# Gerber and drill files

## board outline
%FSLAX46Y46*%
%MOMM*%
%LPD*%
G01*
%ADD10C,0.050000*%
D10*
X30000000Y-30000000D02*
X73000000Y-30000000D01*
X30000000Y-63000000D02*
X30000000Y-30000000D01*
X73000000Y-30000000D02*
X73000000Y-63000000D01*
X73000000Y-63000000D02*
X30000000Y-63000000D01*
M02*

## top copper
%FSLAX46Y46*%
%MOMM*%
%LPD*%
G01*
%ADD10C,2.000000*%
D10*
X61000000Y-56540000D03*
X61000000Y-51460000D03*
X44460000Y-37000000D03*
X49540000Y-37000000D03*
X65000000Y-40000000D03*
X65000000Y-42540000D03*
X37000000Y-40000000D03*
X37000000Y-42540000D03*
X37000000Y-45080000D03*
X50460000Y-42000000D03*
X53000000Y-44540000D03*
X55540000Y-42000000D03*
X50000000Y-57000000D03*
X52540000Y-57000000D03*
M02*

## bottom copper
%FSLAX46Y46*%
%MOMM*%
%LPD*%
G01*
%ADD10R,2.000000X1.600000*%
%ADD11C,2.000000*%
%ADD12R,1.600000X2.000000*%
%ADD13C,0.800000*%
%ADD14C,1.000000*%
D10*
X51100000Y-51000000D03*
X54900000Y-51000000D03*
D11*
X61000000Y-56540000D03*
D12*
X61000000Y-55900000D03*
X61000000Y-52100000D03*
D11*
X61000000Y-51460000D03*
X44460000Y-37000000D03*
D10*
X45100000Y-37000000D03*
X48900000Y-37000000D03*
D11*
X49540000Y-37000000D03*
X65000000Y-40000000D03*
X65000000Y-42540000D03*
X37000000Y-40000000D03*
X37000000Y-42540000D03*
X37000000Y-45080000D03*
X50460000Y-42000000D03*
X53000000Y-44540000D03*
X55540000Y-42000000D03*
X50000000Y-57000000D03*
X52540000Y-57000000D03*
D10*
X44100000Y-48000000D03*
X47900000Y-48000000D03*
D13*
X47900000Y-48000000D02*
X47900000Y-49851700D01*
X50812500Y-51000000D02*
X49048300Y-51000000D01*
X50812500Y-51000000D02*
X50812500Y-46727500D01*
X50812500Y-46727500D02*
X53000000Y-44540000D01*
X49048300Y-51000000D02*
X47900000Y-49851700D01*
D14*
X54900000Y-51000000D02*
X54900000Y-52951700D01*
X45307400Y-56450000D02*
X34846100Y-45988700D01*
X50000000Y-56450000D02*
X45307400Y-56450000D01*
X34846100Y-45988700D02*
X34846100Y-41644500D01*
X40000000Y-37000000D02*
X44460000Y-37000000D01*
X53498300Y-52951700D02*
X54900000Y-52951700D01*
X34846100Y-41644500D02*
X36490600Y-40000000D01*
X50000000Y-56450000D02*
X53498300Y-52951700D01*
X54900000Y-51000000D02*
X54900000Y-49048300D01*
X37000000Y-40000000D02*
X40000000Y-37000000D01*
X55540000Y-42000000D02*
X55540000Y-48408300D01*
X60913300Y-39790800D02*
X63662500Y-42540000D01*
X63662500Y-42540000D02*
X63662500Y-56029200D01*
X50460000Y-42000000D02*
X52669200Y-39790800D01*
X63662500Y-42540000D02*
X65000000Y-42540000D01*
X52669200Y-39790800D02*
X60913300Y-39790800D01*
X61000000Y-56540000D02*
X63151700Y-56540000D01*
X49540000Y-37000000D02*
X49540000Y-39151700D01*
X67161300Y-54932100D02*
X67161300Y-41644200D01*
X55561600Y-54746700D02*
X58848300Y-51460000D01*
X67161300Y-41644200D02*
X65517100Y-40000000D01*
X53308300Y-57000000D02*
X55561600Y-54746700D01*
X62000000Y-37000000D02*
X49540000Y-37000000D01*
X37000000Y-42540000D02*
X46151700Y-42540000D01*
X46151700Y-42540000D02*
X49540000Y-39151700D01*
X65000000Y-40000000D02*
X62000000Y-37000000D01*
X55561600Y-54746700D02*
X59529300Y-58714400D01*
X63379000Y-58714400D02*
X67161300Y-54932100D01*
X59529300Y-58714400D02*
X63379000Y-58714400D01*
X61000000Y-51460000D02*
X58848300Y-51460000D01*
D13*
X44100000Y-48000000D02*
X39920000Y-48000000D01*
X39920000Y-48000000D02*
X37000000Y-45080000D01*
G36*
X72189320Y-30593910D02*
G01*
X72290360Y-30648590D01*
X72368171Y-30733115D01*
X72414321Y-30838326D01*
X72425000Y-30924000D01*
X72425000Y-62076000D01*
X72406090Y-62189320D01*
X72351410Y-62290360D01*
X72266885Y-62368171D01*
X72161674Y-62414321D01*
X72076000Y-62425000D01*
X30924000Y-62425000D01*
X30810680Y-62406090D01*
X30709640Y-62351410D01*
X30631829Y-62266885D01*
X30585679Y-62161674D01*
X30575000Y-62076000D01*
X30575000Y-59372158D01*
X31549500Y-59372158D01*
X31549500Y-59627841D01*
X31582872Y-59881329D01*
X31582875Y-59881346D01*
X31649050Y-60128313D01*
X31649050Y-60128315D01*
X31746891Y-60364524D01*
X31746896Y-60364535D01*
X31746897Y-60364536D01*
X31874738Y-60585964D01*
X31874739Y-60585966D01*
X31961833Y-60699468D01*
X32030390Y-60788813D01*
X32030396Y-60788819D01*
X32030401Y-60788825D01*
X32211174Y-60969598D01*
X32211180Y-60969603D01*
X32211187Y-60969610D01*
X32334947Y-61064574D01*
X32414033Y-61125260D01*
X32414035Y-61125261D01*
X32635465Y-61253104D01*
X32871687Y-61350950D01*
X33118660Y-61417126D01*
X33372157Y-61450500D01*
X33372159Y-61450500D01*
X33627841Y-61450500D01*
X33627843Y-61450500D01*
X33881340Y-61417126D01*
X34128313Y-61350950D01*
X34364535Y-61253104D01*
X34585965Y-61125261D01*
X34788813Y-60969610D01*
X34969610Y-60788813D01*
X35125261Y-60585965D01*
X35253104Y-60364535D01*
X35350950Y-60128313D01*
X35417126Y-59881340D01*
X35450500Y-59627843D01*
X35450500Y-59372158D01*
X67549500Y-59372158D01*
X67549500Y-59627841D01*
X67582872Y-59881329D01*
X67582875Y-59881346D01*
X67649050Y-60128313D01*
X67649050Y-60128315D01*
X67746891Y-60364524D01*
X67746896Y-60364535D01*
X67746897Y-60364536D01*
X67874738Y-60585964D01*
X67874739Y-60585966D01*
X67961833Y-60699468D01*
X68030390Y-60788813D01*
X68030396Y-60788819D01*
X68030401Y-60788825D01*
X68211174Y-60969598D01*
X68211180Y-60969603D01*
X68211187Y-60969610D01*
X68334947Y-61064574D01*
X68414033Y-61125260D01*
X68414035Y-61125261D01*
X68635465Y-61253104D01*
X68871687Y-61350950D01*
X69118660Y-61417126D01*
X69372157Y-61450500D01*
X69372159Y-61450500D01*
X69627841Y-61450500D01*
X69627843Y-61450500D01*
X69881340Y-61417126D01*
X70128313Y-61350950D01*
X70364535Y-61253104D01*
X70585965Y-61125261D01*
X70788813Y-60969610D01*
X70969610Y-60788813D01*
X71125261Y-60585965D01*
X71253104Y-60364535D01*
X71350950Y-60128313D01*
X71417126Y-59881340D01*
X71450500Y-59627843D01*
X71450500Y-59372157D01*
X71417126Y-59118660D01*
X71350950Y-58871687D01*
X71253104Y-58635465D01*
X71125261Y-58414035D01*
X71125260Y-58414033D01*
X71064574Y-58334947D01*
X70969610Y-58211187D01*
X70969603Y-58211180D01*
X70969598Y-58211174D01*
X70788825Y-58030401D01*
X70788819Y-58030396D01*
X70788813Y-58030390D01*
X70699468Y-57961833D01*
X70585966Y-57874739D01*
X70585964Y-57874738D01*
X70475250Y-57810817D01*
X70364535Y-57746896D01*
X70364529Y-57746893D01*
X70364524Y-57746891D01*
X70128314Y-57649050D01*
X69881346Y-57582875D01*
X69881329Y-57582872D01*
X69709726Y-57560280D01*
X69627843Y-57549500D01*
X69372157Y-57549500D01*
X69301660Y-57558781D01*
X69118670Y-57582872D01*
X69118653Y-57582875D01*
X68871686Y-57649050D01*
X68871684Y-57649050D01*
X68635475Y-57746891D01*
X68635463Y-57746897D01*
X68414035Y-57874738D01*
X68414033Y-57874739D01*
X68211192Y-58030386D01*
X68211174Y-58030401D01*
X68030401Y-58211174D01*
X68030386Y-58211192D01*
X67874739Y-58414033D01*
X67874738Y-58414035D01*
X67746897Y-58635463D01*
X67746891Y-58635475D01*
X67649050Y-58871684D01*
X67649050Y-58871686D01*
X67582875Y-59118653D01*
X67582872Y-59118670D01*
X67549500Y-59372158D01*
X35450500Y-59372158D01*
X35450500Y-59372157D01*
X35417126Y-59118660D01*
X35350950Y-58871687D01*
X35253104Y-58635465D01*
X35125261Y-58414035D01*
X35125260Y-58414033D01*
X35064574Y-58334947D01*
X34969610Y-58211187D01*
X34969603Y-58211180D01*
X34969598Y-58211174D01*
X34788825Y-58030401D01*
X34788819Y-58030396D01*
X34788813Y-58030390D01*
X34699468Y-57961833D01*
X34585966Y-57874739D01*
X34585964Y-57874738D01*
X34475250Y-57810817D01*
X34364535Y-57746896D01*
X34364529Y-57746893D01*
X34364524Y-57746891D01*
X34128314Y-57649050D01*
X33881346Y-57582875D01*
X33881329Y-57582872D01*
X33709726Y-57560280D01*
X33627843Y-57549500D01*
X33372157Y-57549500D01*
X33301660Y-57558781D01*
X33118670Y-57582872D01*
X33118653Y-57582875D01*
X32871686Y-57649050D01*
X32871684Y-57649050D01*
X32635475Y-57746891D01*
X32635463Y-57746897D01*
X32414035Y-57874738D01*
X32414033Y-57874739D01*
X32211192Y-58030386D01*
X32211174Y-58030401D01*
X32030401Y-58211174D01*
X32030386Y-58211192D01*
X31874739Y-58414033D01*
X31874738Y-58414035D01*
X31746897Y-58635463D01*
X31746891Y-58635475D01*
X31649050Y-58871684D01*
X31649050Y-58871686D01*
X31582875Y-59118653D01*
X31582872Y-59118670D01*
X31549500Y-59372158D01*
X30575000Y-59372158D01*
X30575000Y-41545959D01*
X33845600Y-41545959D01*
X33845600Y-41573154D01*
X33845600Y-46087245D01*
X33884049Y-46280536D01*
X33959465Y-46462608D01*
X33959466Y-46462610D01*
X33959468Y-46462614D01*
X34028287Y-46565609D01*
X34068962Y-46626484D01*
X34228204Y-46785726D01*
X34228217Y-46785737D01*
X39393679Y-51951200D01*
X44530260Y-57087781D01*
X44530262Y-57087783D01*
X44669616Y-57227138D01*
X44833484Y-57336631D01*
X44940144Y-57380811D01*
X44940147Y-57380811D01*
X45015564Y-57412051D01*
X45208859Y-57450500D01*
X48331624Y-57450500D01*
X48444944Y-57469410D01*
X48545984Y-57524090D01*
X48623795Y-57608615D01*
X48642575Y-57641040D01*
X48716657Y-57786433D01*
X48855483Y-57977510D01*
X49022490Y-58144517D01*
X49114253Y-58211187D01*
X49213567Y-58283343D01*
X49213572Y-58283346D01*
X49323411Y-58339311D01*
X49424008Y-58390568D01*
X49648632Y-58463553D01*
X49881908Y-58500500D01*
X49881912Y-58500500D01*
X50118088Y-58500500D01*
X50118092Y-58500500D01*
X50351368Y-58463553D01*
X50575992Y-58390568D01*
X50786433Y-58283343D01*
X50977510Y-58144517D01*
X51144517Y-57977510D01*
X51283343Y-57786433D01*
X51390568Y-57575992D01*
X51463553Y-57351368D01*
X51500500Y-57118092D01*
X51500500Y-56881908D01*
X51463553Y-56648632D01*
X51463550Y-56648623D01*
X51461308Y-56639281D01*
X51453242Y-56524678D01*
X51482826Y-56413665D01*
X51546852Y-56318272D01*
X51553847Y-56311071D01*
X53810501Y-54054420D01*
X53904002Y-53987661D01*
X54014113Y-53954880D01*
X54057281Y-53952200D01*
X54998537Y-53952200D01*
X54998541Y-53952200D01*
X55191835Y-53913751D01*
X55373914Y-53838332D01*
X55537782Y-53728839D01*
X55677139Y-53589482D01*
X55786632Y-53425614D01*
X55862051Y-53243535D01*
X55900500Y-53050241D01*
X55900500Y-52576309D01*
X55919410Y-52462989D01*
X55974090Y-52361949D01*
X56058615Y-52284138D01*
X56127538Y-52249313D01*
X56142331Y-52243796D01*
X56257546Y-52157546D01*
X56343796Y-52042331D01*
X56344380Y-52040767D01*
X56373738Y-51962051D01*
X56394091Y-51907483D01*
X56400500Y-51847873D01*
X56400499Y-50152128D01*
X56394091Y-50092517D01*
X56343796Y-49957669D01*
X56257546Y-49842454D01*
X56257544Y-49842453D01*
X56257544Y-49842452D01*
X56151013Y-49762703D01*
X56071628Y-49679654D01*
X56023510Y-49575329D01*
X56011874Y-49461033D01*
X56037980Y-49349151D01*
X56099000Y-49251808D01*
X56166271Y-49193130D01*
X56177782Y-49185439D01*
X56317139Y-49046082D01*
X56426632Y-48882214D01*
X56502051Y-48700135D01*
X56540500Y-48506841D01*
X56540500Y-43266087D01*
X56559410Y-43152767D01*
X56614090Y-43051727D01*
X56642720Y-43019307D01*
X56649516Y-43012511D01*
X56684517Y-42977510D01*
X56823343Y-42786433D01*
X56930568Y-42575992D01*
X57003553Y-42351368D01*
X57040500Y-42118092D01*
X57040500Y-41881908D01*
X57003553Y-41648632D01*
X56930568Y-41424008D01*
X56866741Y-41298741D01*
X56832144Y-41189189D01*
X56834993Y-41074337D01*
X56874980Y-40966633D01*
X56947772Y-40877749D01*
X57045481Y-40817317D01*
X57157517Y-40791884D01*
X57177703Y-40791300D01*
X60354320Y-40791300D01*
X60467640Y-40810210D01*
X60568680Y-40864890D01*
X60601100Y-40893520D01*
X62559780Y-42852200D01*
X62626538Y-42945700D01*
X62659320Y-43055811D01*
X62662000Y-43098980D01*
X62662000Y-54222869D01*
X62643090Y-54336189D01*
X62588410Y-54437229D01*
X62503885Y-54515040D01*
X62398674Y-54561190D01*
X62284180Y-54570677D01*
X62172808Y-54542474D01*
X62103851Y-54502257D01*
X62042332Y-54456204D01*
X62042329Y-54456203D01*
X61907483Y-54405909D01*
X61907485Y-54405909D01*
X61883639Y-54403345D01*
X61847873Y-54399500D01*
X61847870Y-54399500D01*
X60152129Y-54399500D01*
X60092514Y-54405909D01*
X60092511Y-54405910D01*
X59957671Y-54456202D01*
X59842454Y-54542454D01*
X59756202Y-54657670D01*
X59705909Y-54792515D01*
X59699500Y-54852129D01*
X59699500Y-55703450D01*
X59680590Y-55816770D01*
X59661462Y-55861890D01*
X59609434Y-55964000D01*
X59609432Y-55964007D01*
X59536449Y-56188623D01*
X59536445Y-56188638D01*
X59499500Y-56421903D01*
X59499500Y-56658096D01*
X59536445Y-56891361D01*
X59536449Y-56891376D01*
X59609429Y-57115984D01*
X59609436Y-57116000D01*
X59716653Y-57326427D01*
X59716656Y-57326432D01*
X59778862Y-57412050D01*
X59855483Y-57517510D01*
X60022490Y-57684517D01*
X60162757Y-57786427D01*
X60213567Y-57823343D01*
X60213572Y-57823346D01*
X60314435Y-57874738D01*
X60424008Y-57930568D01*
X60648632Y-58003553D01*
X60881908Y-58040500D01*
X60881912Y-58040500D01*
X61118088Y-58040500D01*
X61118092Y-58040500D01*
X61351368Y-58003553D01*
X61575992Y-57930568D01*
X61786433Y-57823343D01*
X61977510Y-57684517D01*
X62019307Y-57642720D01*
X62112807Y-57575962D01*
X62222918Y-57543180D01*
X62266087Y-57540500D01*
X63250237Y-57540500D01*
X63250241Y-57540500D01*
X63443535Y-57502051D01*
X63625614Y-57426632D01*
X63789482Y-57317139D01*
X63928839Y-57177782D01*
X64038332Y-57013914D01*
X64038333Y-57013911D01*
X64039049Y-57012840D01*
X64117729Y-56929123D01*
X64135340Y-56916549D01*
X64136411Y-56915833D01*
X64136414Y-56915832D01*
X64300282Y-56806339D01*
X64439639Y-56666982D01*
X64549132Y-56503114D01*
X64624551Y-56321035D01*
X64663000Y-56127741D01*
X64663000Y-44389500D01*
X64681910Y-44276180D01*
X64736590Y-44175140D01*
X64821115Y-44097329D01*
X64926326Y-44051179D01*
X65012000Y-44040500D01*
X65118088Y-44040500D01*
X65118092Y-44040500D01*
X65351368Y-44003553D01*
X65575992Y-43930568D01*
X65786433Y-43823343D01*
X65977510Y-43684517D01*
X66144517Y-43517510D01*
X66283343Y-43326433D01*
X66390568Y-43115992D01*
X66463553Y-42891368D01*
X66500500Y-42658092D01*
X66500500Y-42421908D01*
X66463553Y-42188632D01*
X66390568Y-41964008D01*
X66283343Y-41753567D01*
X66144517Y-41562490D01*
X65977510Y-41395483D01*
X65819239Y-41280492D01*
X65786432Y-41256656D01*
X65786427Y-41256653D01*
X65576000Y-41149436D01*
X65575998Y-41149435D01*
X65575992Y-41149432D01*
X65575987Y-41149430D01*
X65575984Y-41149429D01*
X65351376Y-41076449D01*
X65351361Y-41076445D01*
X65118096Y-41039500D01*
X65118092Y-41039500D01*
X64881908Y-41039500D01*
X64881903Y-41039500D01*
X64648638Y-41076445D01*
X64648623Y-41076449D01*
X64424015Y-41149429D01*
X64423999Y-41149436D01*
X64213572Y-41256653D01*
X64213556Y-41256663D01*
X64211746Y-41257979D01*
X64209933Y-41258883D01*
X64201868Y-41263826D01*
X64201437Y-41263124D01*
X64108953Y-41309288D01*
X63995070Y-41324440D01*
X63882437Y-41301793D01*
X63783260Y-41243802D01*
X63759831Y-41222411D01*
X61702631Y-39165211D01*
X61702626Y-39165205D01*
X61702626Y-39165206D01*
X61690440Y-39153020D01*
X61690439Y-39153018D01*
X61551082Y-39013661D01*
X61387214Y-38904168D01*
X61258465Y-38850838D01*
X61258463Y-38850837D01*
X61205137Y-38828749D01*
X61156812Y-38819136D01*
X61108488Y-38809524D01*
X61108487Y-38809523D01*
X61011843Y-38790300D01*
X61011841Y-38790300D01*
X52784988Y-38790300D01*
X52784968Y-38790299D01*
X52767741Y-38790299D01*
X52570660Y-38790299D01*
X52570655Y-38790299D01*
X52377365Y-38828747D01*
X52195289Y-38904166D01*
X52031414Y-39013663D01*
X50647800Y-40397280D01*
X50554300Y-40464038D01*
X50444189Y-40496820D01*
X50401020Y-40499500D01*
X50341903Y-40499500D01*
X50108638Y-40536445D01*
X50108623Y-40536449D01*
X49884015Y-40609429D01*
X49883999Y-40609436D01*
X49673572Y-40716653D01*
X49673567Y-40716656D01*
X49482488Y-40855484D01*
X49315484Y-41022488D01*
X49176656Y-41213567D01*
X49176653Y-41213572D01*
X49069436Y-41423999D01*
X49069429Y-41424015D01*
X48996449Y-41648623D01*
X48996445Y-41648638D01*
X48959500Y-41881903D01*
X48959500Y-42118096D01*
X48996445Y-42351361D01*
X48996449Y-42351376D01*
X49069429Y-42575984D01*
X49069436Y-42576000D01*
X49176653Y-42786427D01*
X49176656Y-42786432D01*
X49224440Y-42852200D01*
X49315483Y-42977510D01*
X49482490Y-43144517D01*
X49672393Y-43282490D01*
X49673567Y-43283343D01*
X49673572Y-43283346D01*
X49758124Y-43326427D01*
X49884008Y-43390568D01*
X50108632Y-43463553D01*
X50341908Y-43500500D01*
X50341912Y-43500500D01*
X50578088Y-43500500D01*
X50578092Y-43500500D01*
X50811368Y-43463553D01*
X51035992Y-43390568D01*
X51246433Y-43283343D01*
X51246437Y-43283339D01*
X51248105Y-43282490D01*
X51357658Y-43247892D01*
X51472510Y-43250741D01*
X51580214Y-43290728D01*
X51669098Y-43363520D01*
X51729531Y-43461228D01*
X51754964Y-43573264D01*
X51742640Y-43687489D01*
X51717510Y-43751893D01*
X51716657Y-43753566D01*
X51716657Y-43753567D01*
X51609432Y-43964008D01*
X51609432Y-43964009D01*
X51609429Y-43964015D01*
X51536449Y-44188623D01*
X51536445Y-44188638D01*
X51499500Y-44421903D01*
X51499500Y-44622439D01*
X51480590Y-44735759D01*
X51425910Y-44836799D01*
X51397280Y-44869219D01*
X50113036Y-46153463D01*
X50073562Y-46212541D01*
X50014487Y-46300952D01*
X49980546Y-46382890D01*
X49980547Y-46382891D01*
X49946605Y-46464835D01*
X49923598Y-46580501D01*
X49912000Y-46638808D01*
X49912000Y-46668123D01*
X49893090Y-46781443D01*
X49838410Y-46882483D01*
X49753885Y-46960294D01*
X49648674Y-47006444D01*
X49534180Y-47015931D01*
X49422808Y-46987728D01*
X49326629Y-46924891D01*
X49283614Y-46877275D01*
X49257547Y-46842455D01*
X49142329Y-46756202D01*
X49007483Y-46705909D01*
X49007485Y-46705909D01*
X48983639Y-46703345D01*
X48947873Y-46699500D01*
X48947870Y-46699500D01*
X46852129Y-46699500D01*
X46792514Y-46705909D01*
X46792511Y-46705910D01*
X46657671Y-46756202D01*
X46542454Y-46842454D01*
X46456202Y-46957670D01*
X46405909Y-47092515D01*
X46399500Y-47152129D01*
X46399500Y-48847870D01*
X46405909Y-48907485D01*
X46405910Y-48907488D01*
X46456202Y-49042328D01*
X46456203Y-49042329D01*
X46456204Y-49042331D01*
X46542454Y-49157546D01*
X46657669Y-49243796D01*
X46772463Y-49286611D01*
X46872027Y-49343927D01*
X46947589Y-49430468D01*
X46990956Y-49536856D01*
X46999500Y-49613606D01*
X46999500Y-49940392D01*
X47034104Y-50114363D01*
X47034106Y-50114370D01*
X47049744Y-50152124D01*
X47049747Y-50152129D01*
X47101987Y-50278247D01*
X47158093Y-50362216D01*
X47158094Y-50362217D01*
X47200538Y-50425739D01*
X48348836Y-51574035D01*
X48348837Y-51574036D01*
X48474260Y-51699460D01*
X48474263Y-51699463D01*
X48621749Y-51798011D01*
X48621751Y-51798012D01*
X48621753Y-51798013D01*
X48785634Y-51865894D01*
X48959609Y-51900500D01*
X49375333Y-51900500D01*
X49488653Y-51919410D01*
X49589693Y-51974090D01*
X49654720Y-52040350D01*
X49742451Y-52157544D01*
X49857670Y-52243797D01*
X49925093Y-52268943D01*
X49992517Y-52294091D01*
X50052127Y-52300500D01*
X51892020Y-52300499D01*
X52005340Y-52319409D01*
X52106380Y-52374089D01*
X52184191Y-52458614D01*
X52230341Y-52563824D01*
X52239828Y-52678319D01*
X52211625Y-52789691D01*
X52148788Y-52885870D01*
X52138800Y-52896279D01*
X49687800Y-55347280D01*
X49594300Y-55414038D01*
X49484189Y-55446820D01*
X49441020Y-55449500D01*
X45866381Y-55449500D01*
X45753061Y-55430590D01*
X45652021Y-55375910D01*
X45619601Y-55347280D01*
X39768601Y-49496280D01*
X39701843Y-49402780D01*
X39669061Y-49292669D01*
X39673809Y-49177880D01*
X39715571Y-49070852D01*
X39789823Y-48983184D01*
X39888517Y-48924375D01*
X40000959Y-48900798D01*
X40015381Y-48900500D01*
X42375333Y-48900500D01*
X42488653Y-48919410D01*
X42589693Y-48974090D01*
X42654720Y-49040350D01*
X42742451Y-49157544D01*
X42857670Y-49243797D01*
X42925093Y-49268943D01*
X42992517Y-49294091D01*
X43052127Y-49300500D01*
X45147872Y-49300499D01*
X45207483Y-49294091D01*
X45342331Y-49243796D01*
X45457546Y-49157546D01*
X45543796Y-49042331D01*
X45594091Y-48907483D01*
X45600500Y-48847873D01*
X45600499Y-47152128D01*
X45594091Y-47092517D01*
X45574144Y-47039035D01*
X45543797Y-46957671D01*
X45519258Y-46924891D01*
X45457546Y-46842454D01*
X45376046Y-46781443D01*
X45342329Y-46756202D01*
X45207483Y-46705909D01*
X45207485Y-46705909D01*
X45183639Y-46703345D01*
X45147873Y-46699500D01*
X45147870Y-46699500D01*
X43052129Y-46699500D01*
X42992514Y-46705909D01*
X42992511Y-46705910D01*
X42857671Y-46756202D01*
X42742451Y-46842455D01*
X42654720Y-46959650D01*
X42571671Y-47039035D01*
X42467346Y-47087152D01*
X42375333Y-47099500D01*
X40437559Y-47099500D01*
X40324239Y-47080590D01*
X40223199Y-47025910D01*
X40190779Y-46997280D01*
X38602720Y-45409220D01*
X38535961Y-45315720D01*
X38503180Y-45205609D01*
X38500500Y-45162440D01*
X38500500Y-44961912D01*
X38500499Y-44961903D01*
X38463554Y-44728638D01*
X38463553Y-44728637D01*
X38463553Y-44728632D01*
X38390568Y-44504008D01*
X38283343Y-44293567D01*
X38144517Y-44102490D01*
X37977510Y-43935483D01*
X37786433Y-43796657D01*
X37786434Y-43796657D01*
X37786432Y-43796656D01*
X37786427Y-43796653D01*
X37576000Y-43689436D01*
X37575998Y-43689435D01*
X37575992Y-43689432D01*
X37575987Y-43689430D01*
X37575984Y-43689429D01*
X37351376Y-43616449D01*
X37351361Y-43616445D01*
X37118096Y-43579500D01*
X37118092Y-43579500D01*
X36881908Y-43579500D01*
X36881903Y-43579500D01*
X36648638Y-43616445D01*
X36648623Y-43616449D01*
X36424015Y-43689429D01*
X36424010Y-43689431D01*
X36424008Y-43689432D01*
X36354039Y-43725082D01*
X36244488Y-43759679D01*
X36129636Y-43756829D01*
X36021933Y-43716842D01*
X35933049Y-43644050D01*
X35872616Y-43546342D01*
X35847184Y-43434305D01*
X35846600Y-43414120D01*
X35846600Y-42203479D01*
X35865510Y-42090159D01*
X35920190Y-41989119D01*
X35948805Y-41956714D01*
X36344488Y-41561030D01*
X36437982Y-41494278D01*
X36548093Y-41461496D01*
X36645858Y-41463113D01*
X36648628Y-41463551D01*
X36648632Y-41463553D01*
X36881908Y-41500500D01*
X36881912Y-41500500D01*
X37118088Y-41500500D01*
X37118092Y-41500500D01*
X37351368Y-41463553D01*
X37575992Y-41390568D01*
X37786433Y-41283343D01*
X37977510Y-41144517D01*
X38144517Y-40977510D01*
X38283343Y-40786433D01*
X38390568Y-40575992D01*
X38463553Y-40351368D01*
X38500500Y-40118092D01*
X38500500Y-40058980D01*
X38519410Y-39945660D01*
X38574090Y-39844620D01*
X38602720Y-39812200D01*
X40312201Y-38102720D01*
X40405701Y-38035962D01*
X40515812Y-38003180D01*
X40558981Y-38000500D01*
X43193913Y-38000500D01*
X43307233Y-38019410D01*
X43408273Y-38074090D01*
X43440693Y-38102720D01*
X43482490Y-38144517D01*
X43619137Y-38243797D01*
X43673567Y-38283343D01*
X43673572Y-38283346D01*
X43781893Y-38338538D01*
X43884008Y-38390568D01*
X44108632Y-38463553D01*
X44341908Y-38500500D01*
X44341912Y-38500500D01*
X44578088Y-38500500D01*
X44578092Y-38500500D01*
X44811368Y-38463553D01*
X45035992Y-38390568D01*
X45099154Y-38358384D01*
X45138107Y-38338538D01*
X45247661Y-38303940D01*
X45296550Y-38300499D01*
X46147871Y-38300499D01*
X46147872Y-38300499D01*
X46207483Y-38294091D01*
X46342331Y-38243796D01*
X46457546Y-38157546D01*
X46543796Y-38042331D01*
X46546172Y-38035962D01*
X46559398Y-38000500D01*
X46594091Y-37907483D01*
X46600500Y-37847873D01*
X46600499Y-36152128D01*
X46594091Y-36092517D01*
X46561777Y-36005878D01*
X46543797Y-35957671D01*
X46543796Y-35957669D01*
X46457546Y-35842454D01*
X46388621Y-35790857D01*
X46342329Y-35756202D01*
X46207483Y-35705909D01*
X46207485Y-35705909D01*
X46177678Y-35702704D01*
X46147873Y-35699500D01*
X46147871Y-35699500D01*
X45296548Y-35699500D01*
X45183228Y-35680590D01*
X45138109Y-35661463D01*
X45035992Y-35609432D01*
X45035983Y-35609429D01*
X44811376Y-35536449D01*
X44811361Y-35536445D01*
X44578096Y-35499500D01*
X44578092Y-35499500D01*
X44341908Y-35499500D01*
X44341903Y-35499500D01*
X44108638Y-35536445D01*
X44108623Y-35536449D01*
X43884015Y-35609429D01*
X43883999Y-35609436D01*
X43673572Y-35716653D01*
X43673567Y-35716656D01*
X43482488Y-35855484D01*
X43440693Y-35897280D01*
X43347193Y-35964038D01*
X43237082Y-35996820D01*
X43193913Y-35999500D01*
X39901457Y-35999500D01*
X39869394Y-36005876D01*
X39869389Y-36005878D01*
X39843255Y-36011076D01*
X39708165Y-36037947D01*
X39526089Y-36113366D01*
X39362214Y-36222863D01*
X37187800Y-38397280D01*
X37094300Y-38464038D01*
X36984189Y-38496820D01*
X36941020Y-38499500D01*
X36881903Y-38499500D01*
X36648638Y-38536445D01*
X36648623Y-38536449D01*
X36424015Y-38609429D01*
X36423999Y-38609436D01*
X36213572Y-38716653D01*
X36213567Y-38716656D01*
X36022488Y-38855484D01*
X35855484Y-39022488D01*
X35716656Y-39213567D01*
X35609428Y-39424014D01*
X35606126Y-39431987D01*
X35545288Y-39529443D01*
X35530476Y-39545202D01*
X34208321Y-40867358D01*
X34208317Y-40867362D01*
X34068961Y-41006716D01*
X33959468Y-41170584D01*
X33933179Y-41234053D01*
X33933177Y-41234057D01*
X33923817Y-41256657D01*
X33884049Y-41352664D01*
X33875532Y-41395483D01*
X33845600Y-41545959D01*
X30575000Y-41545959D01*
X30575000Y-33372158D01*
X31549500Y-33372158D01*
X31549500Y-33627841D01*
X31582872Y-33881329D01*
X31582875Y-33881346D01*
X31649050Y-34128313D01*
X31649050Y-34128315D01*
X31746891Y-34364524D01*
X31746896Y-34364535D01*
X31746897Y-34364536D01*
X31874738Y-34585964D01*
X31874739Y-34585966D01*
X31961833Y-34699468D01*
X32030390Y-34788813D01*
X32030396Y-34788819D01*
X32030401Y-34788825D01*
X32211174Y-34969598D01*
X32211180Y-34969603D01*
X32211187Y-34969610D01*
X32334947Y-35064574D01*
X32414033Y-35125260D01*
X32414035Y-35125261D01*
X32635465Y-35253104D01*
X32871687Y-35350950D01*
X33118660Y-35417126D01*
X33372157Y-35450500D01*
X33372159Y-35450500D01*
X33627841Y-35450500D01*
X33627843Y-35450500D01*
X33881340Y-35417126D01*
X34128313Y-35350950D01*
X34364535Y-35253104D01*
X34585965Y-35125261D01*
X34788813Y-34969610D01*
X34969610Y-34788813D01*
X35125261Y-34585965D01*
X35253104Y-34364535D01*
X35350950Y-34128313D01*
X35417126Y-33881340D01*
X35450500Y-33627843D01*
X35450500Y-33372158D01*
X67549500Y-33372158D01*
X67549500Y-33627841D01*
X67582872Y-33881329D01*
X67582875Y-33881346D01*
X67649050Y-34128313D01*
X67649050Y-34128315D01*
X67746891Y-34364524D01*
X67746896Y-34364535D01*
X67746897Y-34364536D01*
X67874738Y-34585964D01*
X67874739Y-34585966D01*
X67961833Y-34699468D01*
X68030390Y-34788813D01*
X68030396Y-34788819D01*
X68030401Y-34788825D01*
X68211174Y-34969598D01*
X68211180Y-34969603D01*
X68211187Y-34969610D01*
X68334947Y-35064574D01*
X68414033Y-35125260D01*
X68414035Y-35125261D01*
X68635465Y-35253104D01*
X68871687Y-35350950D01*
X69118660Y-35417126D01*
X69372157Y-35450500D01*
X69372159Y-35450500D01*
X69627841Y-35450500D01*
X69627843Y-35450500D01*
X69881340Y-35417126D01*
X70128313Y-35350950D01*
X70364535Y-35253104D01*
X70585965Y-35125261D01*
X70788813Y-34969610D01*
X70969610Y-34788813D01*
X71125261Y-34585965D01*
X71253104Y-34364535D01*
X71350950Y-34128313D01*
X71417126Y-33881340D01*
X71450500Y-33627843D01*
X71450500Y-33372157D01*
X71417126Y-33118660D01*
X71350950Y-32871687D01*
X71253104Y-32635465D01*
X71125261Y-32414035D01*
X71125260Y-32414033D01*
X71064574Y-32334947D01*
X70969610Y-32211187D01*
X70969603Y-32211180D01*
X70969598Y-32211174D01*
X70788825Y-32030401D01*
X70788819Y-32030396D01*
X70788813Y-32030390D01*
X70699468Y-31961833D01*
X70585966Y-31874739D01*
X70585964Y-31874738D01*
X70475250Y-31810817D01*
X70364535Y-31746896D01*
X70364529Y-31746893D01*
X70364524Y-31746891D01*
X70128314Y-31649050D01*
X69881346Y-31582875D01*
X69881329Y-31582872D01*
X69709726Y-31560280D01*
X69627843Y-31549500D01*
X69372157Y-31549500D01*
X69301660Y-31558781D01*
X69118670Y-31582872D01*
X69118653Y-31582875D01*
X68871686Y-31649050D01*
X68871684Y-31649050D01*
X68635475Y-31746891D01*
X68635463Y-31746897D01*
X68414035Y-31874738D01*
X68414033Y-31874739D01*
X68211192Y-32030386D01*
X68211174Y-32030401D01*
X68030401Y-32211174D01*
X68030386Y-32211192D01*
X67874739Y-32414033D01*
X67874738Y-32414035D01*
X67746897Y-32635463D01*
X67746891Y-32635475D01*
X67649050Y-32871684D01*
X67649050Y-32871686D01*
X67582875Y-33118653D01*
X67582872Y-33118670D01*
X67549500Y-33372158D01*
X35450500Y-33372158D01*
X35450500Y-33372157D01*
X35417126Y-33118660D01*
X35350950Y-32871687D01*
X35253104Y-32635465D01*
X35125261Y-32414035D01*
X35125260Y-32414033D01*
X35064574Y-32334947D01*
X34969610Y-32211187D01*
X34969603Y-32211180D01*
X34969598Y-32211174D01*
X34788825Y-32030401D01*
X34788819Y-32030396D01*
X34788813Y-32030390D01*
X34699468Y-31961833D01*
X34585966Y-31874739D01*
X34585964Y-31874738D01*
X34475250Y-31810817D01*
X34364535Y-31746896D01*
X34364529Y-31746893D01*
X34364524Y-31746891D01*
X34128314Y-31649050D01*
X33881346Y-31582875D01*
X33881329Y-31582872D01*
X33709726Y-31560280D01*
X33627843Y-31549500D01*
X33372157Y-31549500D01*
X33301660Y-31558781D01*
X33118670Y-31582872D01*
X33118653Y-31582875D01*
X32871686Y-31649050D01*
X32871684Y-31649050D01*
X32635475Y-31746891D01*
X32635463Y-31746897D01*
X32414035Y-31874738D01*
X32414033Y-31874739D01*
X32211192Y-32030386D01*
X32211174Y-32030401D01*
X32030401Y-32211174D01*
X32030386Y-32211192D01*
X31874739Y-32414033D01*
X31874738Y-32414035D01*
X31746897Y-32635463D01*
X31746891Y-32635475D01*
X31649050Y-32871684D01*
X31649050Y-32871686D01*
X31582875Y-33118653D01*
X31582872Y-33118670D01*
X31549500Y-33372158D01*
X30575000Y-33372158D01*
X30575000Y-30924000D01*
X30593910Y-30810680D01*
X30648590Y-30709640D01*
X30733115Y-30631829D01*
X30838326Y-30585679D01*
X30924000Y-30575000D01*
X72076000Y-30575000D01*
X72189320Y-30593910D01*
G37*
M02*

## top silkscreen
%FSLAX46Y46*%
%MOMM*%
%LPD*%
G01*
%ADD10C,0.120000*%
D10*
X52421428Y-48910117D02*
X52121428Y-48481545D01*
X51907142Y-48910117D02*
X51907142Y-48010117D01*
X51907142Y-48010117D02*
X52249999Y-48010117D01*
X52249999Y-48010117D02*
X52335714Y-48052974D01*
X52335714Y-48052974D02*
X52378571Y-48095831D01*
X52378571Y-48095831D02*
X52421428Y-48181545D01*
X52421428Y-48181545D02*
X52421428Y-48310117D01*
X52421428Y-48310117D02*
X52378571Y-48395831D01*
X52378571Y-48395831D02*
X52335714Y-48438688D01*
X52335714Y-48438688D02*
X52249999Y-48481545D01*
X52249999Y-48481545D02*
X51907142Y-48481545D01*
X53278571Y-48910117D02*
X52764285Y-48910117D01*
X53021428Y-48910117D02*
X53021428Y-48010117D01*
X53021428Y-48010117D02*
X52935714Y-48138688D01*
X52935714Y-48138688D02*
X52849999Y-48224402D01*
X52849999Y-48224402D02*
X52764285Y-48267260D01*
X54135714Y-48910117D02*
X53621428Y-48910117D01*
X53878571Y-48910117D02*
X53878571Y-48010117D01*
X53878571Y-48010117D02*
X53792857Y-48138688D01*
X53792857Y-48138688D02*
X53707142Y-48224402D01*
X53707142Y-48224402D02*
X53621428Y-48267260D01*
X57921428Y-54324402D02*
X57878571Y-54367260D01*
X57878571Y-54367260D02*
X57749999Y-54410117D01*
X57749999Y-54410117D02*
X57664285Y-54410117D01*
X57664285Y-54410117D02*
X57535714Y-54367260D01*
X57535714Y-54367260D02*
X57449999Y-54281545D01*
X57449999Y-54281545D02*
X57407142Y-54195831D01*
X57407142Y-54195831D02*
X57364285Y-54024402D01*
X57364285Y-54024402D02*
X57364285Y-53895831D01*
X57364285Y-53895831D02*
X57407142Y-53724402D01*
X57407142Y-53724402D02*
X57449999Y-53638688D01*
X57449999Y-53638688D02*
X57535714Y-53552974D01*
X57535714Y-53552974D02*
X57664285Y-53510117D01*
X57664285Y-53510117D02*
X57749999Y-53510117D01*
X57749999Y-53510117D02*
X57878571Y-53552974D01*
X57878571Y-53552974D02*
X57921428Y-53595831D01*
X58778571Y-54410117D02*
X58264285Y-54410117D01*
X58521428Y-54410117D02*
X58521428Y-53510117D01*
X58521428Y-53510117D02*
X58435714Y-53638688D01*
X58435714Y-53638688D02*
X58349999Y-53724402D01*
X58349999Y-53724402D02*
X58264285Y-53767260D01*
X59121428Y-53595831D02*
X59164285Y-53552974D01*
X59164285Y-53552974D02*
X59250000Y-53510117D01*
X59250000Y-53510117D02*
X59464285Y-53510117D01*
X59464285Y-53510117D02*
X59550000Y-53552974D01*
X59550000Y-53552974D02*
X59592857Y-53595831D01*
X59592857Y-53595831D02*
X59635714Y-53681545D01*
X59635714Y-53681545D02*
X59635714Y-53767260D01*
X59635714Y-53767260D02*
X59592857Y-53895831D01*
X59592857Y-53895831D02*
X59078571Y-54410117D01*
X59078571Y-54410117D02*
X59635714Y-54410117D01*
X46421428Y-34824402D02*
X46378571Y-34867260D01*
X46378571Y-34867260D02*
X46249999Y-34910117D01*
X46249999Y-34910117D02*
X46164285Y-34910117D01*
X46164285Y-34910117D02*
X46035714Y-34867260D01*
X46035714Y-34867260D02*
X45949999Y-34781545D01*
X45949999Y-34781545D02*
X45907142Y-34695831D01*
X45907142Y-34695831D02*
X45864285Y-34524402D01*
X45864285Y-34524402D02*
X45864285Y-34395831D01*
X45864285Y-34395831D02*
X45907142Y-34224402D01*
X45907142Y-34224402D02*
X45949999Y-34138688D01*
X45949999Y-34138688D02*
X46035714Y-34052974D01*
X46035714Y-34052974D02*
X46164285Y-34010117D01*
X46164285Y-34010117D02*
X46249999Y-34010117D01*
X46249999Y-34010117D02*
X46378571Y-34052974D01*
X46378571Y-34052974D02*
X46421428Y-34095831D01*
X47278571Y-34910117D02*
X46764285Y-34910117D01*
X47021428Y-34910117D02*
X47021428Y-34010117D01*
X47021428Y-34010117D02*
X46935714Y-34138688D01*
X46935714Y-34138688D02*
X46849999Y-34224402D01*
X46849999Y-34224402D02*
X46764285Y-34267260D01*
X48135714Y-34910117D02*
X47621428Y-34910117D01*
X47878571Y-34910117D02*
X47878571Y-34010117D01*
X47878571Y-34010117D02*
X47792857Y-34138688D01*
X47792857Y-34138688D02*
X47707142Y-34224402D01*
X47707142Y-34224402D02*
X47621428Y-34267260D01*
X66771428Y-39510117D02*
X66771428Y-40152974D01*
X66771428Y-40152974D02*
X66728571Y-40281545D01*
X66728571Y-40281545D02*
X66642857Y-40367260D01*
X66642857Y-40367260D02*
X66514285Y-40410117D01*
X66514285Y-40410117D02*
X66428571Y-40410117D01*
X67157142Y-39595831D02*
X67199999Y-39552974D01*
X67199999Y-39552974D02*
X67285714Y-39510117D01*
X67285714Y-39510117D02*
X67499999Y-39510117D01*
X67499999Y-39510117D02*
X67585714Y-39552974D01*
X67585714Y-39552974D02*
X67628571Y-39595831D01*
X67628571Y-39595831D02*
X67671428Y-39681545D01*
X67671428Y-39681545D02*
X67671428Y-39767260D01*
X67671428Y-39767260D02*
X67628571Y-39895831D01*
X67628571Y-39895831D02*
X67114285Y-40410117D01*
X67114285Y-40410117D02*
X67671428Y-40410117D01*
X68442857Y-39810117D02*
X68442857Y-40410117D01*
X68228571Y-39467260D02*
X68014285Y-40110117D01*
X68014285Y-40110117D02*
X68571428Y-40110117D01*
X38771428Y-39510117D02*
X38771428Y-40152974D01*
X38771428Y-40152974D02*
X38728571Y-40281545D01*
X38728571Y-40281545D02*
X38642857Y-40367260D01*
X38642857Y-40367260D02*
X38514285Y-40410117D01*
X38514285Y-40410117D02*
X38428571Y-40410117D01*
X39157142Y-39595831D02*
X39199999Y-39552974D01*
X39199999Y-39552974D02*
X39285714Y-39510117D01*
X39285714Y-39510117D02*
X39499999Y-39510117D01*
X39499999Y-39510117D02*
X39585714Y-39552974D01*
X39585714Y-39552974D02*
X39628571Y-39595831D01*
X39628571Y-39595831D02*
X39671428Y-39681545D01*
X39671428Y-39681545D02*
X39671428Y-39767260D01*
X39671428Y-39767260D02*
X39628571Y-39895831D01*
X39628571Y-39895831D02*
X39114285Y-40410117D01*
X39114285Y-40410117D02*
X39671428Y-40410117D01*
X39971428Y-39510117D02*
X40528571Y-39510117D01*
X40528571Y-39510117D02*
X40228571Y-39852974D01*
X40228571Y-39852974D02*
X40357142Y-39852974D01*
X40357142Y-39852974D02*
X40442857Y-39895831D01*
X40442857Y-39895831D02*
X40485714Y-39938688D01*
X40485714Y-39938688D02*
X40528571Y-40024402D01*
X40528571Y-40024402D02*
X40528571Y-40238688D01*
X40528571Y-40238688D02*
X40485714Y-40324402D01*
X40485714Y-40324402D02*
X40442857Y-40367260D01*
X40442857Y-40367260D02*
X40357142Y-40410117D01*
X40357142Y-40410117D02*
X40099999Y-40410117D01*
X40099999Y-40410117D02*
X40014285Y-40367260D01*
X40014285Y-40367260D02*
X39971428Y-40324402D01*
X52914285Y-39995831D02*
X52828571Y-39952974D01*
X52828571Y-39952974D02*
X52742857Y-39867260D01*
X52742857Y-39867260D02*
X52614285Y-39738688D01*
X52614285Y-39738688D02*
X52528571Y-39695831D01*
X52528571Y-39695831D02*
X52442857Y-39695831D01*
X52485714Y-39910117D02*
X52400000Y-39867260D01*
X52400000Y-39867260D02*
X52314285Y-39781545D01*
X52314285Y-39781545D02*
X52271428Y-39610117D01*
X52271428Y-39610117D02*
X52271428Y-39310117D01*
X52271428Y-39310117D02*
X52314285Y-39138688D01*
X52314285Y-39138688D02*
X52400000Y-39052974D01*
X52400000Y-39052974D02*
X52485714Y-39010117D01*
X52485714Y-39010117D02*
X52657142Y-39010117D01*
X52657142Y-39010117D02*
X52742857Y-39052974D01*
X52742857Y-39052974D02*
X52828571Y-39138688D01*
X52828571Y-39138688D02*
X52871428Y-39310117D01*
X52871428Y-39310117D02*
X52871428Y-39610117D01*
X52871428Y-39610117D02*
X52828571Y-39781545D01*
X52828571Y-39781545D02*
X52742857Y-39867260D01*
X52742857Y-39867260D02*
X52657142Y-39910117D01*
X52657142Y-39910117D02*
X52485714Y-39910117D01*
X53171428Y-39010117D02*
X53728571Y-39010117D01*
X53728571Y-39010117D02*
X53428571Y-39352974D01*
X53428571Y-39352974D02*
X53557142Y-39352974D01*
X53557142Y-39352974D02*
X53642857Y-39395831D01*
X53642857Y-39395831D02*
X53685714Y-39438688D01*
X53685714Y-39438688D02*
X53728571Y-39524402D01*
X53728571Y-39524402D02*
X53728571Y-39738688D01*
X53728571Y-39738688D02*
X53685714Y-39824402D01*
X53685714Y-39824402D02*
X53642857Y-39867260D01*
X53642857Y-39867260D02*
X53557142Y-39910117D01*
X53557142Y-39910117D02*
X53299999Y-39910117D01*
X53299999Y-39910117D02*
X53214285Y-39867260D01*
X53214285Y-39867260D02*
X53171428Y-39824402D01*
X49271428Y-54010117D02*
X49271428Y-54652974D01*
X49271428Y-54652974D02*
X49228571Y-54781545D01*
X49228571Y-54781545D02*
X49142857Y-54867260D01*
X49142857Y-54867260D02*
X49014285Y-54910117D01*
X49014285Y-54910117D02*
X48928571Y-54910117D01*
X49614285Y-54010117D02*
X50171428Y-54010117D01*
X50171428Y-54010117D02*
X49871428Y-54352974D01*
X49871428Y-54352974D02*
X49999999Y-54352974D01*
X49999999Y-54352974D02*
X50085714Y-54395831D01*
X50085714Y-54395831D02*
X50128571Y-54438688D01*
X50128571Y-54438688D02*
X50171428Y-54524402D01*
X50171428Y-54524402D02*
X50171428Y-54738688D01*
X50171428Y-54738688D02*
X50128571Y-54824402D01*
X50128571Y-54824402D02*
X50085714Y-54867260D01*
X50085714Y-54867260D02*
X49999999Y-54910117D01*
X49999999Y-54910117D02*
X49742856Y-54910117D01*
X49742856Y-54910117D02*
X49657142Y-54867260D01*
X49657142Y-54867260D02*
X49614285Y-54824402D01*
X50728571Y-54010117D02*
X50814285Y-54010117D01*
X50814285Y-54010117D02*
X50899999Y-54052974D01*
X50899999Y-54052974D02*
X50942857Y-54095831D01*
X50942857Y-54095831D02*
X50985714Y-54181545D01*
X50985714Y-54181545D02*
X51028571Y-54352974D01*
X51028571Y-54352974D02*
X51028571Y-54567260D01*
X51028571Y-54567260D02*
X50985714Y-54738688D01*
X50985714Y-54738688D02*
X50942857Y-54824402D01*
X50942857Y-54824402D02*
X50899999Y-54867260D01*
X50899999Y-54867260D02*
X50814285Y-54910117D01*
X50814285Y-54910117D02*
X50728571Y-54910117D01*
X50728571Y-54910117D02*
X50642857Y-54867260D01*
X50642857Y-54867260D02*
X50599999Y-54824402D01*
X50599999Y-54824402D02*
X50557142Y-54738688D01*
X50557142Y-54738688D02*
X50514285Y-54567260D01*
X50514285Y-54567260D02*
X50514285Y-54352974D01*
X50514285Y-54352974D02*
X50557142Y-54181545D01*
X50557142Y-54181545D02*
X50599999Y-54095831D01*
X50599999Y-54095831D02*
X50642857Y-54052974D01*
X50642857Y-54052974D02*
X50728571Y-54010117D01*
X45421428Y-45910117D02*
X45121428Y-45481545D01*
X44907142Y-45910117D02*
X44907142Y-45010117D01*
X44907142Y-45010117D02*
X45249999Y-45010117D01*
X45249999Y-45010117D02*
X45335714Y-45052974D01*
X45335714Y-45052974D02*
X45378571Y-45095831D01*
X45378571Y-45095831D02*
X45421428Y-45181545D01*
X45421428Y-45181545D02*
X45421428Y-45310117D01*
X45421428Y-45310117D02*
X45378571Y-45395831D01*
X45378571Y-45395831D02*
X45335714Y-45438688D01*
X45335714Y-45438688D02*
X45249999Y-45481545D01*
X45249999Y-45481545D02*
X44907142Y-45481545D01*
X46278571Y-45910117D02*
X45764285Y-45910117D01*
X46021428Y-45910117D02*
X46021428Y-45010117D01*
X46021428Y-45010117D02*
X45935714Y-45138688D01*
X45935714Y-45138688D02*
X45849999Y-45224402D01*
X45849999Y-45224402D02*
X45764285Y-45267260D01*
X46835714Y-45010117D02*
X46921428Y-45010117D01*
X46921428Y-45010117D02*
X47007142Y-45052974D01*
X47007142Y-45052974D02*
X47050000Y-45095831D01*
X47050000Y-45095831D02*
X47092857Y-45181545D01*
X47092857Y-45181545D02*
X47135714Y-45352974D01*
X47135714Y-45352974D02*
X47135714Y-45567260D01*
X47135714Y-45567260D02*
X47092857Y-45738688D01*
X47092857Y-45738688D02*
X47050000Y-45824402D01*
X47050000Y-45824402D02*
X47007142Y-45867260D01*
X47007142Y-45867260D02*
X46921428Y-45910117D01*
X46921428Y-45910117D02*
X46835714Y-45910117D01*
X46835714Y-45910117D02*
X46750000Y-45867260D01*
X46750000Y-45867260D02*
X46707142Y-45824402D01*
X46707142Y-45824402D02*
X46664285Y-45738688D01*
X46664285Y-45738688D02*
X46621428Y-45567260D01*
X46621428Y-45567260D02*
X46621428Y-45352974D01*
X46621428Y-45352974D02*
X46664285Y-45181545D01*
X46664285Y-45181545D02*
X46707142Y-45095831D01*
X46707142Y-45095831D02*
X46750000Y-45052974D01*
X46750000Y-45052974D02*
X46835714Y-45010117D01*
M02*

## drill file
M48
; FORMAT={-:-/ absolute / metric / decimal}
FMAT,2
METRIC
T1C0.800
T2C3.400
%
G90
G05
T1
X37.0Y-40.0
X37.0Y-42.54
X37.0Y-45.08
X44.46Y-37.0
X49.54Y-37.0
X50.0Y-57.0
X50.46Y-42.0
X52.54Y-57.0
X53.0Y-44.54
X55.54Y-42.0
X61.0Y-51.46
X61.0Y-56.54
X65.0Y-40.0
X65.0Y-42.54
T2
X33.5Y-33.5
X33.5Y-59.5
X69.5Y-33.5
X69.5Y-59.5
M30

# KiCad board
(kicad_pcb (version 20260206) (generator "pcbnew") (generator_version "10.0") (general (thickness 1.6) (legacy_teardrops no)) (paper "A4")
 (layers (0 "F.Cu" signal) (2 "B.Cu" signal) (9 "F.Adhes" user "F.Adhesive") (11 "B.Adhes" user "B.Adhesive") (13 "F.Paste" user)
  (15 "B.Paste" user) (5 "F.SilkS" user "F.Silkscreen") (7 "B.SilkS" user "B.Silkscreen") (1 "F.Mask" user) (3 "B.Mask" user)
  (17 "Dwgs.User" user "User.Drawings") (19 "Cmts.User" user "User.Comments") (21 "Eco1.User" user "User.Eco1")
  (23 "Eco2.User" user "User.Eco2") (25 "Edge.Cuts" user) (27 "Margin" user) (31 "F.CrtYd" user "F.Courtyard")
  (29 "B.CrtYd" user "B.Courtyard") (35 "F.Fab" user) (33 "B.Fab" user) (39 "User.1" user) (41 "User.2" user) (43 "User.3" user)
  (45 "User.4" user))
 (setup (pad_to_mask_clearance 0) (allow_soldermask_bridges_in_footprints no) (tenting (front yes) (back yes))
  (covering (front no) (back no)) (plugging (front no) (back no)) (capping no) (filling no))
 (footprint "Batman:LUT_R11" (layer "F.Cu") (at 53 51)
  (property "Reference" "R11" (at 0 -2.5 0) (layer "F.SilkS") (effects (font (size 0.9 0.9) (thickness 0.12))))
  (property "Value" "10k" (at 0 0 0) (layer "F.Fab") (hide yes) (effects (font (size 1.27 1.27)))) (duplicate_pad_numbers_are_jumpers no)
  (pad "1" smd rect (at -1.9 0) (size 2 1.6) (layers "B.Cu") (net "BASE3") (thermal_bridge_angle 45))
  (pad "2" smd rect (at 1.9 0) (size 2 1.6) (layers "B.Cu") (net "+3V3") (thermal_bridge_angle 45)))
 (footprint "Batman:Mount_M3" (layer "F.Cu") (at 69.5 33.5)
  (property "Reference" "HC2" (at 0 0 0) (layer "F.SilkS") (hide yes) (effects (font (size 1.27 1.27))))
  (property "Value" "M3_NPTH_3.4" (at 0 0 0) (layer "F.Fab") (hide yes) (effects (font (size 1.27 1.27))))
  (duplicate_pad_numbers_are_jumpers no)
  (pad "" np_thru_hole circle (at 0 0) (size 3.4 3.4) (drill 3.4) (layers "*.Cu")))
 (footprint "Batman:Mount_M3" (layer "F.Cu") (at 33.5 59.5)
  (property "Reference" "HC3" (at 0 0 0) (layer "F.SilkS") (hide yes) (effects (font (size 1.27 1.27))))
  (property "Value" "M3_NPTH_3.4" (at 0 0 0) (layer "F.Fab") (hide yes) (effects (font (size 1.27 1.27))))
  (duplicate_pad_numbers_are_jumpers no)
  (pad "" np_thru_hole circle (at 0 0) (size 3.4 3.4) (drill 3.4) (layers "*.Cu")))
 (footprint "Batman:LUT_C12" (layer "F.Cu") (at 61 54 90)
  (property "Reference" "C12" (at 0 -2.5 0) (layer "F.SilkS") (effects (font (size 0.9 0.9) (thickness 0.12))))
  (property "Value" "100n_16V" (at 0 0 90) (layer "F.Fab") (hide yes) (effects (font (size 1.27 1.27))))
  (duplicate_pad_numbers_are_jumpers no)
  (pad "1" thru_hole circle (at -2.54 0 90) (size 2 2) (drill 0.8) (layers "*.Cu") (remove_unused_layers no) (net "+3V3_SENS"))
  (pad "1" smd rect (at -1.9 0 90) (size 2 1.6) (layers "B.Cu") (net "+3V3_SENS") (thermal_bridge_angle 45))
  (pad "2" smd rect (at 1.9 0 90) (size 2 1.6) (layers "B.Cu") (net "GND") (thermal_bridge_angle 45))
  (pad "2" thru_hole circle (at 2.54 0 90) (size 2 2) (drill 0.8) (layers "*.Cu") (remove_unused_layers no) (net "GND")))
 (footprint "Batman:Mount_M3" (layer "F.Cu") (at 33.5 33.5)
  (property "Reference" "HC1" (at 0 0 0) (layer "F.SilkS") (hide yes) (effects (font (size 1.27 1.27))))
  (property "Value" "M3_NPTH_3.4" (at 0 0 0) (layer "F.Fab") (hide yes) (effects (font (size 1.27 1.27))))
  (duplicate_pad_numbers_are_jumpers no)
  (pad "" np_thru_hole circle (at 0 0) (size 3.4 3.4) (drill 3.4) (layers "*.Cu")))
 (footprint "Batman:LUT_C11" (layer "F.Cu") (at 47 37)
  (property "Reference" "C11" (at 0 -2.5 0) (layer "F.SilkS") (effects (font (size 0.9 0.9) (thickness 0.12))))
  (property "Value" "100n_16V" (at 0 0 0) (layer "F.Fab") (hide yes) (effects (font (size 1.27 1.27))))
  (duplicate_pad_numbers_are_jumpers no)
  (pad "1" thru_hole circle (at -2.54 0) (size 2 2) (drill 0.8) (layers "*.Cu") (remove_unused_layers no) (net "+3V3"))
  (pad "1" smd rect (at -1.9 0) (size 2 1.6) (layers "B.Cu") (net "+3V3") (thermal_bridge_angle 45))
  (pad "2" smd rect (at 1.9 0) (size 2 1.6) (layers "B.Cu") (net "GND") (thermal_bridge_angle 45))
  (pad "2" thru_hole circle (at 2.54 0) (size 2 2) (drill 0.8) (layers "*.Cu") (remove_unused_layers no) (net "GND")))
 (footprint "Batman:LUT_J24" (layer "F.Cu") (at 65 40 -90)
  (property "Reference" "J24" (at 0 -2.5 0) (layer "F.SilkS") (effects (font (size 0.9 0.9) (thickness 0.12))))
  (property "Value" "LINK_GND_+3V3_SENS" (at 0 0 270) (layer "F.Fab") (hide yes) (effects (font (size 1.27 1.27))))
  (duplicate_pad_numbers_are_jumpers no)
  (pad "1" thru_hole circle (at 0 0 270) (size 2 2) (drill 0.8) (layers "*.Cu") (remove_unused_layers no) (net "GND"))
  (pad "2" thru_hole circle (at 2.54 0 270) (size 2 2) (drill 0.8) (layers "*.Cu") (remove_unused_layers no) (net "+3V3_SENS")))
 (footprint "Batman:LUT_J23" (layer "F.Cu") (at 37 40 -90)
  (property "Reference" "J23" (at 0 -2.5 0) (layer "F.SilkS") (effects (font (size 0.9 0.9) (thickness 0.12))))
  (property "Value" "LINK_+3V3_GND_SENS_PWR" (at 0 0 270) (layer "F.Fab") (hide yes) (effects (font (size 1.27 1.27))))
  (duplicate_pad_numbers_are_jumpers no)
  (pad "1" thru_hole circle (at 0 0 270) (size 2 2) (drill 0.8) (layers "*.Cu") (remove_unused_layers no) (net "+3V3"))
  (pad "2" thru_hole circle (at 2.54 0 270) (size 2 2) (drill 0.8) (layers "*.Cu") (remove_unused_layers no) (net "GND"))
  (pad "3" thru_hole circle (at 5.08 0 270) (size 2 2) (drill 0.8) (layers "*.Cu") (remove_unused_layers no) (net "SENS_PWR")))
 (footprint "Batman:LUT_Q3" (layer "F.Cu") (at 53 42)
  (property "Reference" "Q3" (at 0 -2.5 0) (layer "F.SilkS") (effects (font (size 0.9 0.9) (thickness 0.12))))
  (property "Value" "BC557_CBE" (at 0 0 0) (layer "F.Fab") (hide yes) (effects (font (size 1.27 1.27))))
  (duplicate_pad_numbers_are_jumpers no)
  (pad "1" thru_hole circle (at -2.54 0) (size 2 2) (drill 0.8) (layers "*.Cu") (remove_unused_layers no) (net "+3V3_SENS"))
  (pad "2" thru_hole circle (at 0 2.54) (size 2 2) (drill 0.8) (layers "*.Cu") (remove_unused_layers no) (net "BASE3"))
  (pad "3" thru_hole circle (at 2.54 0) (size 2 2) (drill 0.8) (layers "*.Cu") (remove_unused_layers no) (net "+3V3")))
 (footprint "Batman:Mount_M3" (layer "F.Cu") (at 69.5 59.5)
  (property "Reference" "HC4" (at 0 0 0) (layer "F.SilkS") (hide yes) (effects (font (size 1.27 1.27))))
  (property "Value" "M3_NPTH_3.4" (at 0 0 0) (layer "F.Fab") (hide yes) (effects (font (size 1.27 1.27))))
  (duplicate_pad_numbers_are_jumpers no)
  (pad "" np_thru_hole circle (at 0 0) (size 3.4 3.4) (drill 3.4) (layers "*.Cu")))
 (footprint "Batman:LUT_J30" (layer "F.Cu") (at 50 57)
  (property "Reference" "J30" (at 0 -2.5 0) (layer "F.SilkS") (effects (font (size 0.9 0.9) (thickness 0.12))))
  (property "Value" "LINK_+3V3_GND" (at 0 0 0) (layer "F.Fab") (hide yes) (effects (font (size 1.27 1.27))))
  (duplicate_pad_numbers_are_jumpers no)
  (pad "1" thru_hole circle (at 0 0) (size 2 2) (drill 0.8) (layers "*.Cu") (remove_unused_layers no) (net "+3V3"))
  (pad "2" thru_hole circle (at 2.54 0) (size 2 2) (drill 0.8) (layers "*.Cu") (remove_unused_layers no) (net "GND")))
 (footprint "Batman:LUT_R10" (layer "F.Cu") (at 46 48)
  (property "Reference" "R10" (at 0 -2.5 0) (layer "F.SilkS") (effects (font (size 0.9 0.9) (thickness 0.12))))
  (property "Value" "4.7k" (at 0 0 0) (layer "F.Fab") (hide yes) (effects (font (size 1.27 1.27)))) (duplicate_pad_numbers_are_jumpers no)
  (pad "1" smd rect (at -1.9 0) (size 2 1.6) (layers "B.Cu") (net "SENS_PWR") (thermal_bridge_angle 45))
  (pad "2" smd rect (at 1.9 0) (size 2 1.6) (layers "B.Cu") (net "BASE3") (thermal_bridge_angle 45)))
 (gr_line (start 30 30) (end 73 30) (stroke (width 0.05) (type default)) (layer "Edge.Cuts"))
 (gr_line (start 30 63) (end 30 30) (stroke (width 0.05) (type default)) (layer "Edge.Cuts"))
 (gr_line (start 73 30) (end 73 63) (stroke (width 0.05) (type default)) (layer "Edge.Cuts"))
 (gr_line (start 73 63) (end 30 63) (stroke (width 0.05) (type default)) (layer "Edge.Cuts"))
 (segment (start 47.9 48) (end 47.9 49.8517) (width 0.8) (layer "B.Cu") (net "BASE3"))
 (segment (start 50.8125 51) (end 49.0483 51) (width 0.8) (layer "B.Cu") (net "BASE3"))
 (segment (start 50.8125 51) (end 50.8125 46.7275) (width 0.8) (layer "B.Cu") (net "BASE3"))
 (segment (start 50.8125 46.7275) (end 53 44.54) (width 0.8) (layer "B.Cu") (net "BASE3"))
 (segment (start 49.0483 51) (end 47.9 49.8517) (width 0.8) (layer "B.Cu") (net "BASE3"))
 (segment (start 54.9 51) (end 54.9 52.9517) (width 1) (layer "B.Cu") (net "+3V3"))
 (segment (start 45.3074 56.45) (end 34.8461 45.9887) (width 1) (layer "B.Cu") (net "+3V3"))
 (segment (start 50 56.45) (end 45.3074 56.45) (width 1) (layer "B.Cu") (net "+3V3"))
 (segment (start 34.8461 45.9887) (end 34.8461 41.6445) (width 1) (layer "B.Cu") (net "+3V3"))
 (segment (start 40 37) (end 44.46 37) (width 1) (layer "B.Cu") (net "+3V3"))
 (segment (start 53.4983 52.9517) (end 54.9 52.9517) (width 1) (layer "B.Cu") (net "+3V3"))
 (segment (start 34.8461 41.6445) (end 36.4906 40) (width 1) (layer "B.Cu") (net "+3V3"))
 (segment (start 50 56.45) (end 53.4983 52.9517) (width 1) (layer "B.Cu") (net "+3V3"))
 (segment (start 54.9 51) (end 54.9 49.0483) (width 1) (layer "B.Cu") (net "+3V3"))
 (segment (start 37 40) (end 40 37) (width 1) (layer "B.Cu") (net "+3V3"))
 (segment (start 55.54 42) (end 55.54 48.4083) (width 1) (layer "B.Cu") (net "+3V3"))
 (segment (start 60.9133 39.7908) (end 63.6625 42.54) (width 1) (layer "B.Cu") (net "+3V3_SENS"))
 (segment (start 63.6625 42.54) (end 63.6625 56.0292) (width 1) (layer "B.Cu") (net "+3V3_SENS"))
 (segment (start 50.46 42) (end 52.6692 39.7908) (width 1) (layer "B.Cu") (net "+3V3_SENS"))
 (segment (start 63.6625 42.54) (end 65 42.54) (width 1) (layer "B.Cu") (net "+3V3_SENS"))
 (segment (start 52.6692 39.7908) (end 60.9133 39.7908) (width 1) (layer "B.Cu") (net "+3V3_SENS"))
 (segment (start 61 56.54) (end 63.1517 56.54) (width 1) (layer "B.Cu") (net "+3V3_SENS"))
 (segment (start 49.54 37) (end 49.54 39.1517) (width 1) (layer "B.Cu") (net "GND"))
 (segment (start 67.1613 54.9321) (end 67.1613 41.6442) (width 1) (layer "B.Cu") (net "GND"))
 (segment (start 55.5616 54.7467) (end 58.8483 51.46) (width 1) (layer "B.Cu") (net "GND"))
 (segment (start 67.1613 41.6442) (end 65.5171 40) (width 1) (layer "B.Cu") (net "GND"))
 (segment (start 53.3083 57) (end 55.5616 54.7467) (width 1) (layer "B.Cu") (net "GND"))
 (segment (start 62 37) (end 49.54 37) (width 1) (layer "B.Cu") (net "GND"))
 (segment (start 37 42.54) (end 46.1517 42.54) (width 1) (layer "B.Cu") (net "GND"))
 (segment (start 46.1517 42.54) (end 49.54 39.1517) (width 1) (layer "B.Cu") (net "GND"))
 (segment (start 65 40) (end 62 37) (width 1) (layer "B.Cu") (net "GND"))
 (segment (start 55.5616 54.7467) (end 59.5293 58.7144) (width 1) (layer "B.Cu") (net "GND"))
 (segment (start 63.379 58.7144) (end 67.1613 54.9321) (width 1) (layer "B.Cu") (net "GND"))
 (segment (start 59.5293 58.7144) (end 63.379 58.7144) (width 1) (layer "B.Cu") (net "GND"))
 (segment (start 61 51.46) (end 58.8483 51.46) (width 1) (layer "B.Cu") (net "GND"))
 (segment (start 44.1 48) (end 39.92 48) (width 0.8) (layer "B.Cu") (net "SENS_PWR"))
 (segment (start 39.92 48) (end 37 45.08) (width 0.8) (layer "B.Cu") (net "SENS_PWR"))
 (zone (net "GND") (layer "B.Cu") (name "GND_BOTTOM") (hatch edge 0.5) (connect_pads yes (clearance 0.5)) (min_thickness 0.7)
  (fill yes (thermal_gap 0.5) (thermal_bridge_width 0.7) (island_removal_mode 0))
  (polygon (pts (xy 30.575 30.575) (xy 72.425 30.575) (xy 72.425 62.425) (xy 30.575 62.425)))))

